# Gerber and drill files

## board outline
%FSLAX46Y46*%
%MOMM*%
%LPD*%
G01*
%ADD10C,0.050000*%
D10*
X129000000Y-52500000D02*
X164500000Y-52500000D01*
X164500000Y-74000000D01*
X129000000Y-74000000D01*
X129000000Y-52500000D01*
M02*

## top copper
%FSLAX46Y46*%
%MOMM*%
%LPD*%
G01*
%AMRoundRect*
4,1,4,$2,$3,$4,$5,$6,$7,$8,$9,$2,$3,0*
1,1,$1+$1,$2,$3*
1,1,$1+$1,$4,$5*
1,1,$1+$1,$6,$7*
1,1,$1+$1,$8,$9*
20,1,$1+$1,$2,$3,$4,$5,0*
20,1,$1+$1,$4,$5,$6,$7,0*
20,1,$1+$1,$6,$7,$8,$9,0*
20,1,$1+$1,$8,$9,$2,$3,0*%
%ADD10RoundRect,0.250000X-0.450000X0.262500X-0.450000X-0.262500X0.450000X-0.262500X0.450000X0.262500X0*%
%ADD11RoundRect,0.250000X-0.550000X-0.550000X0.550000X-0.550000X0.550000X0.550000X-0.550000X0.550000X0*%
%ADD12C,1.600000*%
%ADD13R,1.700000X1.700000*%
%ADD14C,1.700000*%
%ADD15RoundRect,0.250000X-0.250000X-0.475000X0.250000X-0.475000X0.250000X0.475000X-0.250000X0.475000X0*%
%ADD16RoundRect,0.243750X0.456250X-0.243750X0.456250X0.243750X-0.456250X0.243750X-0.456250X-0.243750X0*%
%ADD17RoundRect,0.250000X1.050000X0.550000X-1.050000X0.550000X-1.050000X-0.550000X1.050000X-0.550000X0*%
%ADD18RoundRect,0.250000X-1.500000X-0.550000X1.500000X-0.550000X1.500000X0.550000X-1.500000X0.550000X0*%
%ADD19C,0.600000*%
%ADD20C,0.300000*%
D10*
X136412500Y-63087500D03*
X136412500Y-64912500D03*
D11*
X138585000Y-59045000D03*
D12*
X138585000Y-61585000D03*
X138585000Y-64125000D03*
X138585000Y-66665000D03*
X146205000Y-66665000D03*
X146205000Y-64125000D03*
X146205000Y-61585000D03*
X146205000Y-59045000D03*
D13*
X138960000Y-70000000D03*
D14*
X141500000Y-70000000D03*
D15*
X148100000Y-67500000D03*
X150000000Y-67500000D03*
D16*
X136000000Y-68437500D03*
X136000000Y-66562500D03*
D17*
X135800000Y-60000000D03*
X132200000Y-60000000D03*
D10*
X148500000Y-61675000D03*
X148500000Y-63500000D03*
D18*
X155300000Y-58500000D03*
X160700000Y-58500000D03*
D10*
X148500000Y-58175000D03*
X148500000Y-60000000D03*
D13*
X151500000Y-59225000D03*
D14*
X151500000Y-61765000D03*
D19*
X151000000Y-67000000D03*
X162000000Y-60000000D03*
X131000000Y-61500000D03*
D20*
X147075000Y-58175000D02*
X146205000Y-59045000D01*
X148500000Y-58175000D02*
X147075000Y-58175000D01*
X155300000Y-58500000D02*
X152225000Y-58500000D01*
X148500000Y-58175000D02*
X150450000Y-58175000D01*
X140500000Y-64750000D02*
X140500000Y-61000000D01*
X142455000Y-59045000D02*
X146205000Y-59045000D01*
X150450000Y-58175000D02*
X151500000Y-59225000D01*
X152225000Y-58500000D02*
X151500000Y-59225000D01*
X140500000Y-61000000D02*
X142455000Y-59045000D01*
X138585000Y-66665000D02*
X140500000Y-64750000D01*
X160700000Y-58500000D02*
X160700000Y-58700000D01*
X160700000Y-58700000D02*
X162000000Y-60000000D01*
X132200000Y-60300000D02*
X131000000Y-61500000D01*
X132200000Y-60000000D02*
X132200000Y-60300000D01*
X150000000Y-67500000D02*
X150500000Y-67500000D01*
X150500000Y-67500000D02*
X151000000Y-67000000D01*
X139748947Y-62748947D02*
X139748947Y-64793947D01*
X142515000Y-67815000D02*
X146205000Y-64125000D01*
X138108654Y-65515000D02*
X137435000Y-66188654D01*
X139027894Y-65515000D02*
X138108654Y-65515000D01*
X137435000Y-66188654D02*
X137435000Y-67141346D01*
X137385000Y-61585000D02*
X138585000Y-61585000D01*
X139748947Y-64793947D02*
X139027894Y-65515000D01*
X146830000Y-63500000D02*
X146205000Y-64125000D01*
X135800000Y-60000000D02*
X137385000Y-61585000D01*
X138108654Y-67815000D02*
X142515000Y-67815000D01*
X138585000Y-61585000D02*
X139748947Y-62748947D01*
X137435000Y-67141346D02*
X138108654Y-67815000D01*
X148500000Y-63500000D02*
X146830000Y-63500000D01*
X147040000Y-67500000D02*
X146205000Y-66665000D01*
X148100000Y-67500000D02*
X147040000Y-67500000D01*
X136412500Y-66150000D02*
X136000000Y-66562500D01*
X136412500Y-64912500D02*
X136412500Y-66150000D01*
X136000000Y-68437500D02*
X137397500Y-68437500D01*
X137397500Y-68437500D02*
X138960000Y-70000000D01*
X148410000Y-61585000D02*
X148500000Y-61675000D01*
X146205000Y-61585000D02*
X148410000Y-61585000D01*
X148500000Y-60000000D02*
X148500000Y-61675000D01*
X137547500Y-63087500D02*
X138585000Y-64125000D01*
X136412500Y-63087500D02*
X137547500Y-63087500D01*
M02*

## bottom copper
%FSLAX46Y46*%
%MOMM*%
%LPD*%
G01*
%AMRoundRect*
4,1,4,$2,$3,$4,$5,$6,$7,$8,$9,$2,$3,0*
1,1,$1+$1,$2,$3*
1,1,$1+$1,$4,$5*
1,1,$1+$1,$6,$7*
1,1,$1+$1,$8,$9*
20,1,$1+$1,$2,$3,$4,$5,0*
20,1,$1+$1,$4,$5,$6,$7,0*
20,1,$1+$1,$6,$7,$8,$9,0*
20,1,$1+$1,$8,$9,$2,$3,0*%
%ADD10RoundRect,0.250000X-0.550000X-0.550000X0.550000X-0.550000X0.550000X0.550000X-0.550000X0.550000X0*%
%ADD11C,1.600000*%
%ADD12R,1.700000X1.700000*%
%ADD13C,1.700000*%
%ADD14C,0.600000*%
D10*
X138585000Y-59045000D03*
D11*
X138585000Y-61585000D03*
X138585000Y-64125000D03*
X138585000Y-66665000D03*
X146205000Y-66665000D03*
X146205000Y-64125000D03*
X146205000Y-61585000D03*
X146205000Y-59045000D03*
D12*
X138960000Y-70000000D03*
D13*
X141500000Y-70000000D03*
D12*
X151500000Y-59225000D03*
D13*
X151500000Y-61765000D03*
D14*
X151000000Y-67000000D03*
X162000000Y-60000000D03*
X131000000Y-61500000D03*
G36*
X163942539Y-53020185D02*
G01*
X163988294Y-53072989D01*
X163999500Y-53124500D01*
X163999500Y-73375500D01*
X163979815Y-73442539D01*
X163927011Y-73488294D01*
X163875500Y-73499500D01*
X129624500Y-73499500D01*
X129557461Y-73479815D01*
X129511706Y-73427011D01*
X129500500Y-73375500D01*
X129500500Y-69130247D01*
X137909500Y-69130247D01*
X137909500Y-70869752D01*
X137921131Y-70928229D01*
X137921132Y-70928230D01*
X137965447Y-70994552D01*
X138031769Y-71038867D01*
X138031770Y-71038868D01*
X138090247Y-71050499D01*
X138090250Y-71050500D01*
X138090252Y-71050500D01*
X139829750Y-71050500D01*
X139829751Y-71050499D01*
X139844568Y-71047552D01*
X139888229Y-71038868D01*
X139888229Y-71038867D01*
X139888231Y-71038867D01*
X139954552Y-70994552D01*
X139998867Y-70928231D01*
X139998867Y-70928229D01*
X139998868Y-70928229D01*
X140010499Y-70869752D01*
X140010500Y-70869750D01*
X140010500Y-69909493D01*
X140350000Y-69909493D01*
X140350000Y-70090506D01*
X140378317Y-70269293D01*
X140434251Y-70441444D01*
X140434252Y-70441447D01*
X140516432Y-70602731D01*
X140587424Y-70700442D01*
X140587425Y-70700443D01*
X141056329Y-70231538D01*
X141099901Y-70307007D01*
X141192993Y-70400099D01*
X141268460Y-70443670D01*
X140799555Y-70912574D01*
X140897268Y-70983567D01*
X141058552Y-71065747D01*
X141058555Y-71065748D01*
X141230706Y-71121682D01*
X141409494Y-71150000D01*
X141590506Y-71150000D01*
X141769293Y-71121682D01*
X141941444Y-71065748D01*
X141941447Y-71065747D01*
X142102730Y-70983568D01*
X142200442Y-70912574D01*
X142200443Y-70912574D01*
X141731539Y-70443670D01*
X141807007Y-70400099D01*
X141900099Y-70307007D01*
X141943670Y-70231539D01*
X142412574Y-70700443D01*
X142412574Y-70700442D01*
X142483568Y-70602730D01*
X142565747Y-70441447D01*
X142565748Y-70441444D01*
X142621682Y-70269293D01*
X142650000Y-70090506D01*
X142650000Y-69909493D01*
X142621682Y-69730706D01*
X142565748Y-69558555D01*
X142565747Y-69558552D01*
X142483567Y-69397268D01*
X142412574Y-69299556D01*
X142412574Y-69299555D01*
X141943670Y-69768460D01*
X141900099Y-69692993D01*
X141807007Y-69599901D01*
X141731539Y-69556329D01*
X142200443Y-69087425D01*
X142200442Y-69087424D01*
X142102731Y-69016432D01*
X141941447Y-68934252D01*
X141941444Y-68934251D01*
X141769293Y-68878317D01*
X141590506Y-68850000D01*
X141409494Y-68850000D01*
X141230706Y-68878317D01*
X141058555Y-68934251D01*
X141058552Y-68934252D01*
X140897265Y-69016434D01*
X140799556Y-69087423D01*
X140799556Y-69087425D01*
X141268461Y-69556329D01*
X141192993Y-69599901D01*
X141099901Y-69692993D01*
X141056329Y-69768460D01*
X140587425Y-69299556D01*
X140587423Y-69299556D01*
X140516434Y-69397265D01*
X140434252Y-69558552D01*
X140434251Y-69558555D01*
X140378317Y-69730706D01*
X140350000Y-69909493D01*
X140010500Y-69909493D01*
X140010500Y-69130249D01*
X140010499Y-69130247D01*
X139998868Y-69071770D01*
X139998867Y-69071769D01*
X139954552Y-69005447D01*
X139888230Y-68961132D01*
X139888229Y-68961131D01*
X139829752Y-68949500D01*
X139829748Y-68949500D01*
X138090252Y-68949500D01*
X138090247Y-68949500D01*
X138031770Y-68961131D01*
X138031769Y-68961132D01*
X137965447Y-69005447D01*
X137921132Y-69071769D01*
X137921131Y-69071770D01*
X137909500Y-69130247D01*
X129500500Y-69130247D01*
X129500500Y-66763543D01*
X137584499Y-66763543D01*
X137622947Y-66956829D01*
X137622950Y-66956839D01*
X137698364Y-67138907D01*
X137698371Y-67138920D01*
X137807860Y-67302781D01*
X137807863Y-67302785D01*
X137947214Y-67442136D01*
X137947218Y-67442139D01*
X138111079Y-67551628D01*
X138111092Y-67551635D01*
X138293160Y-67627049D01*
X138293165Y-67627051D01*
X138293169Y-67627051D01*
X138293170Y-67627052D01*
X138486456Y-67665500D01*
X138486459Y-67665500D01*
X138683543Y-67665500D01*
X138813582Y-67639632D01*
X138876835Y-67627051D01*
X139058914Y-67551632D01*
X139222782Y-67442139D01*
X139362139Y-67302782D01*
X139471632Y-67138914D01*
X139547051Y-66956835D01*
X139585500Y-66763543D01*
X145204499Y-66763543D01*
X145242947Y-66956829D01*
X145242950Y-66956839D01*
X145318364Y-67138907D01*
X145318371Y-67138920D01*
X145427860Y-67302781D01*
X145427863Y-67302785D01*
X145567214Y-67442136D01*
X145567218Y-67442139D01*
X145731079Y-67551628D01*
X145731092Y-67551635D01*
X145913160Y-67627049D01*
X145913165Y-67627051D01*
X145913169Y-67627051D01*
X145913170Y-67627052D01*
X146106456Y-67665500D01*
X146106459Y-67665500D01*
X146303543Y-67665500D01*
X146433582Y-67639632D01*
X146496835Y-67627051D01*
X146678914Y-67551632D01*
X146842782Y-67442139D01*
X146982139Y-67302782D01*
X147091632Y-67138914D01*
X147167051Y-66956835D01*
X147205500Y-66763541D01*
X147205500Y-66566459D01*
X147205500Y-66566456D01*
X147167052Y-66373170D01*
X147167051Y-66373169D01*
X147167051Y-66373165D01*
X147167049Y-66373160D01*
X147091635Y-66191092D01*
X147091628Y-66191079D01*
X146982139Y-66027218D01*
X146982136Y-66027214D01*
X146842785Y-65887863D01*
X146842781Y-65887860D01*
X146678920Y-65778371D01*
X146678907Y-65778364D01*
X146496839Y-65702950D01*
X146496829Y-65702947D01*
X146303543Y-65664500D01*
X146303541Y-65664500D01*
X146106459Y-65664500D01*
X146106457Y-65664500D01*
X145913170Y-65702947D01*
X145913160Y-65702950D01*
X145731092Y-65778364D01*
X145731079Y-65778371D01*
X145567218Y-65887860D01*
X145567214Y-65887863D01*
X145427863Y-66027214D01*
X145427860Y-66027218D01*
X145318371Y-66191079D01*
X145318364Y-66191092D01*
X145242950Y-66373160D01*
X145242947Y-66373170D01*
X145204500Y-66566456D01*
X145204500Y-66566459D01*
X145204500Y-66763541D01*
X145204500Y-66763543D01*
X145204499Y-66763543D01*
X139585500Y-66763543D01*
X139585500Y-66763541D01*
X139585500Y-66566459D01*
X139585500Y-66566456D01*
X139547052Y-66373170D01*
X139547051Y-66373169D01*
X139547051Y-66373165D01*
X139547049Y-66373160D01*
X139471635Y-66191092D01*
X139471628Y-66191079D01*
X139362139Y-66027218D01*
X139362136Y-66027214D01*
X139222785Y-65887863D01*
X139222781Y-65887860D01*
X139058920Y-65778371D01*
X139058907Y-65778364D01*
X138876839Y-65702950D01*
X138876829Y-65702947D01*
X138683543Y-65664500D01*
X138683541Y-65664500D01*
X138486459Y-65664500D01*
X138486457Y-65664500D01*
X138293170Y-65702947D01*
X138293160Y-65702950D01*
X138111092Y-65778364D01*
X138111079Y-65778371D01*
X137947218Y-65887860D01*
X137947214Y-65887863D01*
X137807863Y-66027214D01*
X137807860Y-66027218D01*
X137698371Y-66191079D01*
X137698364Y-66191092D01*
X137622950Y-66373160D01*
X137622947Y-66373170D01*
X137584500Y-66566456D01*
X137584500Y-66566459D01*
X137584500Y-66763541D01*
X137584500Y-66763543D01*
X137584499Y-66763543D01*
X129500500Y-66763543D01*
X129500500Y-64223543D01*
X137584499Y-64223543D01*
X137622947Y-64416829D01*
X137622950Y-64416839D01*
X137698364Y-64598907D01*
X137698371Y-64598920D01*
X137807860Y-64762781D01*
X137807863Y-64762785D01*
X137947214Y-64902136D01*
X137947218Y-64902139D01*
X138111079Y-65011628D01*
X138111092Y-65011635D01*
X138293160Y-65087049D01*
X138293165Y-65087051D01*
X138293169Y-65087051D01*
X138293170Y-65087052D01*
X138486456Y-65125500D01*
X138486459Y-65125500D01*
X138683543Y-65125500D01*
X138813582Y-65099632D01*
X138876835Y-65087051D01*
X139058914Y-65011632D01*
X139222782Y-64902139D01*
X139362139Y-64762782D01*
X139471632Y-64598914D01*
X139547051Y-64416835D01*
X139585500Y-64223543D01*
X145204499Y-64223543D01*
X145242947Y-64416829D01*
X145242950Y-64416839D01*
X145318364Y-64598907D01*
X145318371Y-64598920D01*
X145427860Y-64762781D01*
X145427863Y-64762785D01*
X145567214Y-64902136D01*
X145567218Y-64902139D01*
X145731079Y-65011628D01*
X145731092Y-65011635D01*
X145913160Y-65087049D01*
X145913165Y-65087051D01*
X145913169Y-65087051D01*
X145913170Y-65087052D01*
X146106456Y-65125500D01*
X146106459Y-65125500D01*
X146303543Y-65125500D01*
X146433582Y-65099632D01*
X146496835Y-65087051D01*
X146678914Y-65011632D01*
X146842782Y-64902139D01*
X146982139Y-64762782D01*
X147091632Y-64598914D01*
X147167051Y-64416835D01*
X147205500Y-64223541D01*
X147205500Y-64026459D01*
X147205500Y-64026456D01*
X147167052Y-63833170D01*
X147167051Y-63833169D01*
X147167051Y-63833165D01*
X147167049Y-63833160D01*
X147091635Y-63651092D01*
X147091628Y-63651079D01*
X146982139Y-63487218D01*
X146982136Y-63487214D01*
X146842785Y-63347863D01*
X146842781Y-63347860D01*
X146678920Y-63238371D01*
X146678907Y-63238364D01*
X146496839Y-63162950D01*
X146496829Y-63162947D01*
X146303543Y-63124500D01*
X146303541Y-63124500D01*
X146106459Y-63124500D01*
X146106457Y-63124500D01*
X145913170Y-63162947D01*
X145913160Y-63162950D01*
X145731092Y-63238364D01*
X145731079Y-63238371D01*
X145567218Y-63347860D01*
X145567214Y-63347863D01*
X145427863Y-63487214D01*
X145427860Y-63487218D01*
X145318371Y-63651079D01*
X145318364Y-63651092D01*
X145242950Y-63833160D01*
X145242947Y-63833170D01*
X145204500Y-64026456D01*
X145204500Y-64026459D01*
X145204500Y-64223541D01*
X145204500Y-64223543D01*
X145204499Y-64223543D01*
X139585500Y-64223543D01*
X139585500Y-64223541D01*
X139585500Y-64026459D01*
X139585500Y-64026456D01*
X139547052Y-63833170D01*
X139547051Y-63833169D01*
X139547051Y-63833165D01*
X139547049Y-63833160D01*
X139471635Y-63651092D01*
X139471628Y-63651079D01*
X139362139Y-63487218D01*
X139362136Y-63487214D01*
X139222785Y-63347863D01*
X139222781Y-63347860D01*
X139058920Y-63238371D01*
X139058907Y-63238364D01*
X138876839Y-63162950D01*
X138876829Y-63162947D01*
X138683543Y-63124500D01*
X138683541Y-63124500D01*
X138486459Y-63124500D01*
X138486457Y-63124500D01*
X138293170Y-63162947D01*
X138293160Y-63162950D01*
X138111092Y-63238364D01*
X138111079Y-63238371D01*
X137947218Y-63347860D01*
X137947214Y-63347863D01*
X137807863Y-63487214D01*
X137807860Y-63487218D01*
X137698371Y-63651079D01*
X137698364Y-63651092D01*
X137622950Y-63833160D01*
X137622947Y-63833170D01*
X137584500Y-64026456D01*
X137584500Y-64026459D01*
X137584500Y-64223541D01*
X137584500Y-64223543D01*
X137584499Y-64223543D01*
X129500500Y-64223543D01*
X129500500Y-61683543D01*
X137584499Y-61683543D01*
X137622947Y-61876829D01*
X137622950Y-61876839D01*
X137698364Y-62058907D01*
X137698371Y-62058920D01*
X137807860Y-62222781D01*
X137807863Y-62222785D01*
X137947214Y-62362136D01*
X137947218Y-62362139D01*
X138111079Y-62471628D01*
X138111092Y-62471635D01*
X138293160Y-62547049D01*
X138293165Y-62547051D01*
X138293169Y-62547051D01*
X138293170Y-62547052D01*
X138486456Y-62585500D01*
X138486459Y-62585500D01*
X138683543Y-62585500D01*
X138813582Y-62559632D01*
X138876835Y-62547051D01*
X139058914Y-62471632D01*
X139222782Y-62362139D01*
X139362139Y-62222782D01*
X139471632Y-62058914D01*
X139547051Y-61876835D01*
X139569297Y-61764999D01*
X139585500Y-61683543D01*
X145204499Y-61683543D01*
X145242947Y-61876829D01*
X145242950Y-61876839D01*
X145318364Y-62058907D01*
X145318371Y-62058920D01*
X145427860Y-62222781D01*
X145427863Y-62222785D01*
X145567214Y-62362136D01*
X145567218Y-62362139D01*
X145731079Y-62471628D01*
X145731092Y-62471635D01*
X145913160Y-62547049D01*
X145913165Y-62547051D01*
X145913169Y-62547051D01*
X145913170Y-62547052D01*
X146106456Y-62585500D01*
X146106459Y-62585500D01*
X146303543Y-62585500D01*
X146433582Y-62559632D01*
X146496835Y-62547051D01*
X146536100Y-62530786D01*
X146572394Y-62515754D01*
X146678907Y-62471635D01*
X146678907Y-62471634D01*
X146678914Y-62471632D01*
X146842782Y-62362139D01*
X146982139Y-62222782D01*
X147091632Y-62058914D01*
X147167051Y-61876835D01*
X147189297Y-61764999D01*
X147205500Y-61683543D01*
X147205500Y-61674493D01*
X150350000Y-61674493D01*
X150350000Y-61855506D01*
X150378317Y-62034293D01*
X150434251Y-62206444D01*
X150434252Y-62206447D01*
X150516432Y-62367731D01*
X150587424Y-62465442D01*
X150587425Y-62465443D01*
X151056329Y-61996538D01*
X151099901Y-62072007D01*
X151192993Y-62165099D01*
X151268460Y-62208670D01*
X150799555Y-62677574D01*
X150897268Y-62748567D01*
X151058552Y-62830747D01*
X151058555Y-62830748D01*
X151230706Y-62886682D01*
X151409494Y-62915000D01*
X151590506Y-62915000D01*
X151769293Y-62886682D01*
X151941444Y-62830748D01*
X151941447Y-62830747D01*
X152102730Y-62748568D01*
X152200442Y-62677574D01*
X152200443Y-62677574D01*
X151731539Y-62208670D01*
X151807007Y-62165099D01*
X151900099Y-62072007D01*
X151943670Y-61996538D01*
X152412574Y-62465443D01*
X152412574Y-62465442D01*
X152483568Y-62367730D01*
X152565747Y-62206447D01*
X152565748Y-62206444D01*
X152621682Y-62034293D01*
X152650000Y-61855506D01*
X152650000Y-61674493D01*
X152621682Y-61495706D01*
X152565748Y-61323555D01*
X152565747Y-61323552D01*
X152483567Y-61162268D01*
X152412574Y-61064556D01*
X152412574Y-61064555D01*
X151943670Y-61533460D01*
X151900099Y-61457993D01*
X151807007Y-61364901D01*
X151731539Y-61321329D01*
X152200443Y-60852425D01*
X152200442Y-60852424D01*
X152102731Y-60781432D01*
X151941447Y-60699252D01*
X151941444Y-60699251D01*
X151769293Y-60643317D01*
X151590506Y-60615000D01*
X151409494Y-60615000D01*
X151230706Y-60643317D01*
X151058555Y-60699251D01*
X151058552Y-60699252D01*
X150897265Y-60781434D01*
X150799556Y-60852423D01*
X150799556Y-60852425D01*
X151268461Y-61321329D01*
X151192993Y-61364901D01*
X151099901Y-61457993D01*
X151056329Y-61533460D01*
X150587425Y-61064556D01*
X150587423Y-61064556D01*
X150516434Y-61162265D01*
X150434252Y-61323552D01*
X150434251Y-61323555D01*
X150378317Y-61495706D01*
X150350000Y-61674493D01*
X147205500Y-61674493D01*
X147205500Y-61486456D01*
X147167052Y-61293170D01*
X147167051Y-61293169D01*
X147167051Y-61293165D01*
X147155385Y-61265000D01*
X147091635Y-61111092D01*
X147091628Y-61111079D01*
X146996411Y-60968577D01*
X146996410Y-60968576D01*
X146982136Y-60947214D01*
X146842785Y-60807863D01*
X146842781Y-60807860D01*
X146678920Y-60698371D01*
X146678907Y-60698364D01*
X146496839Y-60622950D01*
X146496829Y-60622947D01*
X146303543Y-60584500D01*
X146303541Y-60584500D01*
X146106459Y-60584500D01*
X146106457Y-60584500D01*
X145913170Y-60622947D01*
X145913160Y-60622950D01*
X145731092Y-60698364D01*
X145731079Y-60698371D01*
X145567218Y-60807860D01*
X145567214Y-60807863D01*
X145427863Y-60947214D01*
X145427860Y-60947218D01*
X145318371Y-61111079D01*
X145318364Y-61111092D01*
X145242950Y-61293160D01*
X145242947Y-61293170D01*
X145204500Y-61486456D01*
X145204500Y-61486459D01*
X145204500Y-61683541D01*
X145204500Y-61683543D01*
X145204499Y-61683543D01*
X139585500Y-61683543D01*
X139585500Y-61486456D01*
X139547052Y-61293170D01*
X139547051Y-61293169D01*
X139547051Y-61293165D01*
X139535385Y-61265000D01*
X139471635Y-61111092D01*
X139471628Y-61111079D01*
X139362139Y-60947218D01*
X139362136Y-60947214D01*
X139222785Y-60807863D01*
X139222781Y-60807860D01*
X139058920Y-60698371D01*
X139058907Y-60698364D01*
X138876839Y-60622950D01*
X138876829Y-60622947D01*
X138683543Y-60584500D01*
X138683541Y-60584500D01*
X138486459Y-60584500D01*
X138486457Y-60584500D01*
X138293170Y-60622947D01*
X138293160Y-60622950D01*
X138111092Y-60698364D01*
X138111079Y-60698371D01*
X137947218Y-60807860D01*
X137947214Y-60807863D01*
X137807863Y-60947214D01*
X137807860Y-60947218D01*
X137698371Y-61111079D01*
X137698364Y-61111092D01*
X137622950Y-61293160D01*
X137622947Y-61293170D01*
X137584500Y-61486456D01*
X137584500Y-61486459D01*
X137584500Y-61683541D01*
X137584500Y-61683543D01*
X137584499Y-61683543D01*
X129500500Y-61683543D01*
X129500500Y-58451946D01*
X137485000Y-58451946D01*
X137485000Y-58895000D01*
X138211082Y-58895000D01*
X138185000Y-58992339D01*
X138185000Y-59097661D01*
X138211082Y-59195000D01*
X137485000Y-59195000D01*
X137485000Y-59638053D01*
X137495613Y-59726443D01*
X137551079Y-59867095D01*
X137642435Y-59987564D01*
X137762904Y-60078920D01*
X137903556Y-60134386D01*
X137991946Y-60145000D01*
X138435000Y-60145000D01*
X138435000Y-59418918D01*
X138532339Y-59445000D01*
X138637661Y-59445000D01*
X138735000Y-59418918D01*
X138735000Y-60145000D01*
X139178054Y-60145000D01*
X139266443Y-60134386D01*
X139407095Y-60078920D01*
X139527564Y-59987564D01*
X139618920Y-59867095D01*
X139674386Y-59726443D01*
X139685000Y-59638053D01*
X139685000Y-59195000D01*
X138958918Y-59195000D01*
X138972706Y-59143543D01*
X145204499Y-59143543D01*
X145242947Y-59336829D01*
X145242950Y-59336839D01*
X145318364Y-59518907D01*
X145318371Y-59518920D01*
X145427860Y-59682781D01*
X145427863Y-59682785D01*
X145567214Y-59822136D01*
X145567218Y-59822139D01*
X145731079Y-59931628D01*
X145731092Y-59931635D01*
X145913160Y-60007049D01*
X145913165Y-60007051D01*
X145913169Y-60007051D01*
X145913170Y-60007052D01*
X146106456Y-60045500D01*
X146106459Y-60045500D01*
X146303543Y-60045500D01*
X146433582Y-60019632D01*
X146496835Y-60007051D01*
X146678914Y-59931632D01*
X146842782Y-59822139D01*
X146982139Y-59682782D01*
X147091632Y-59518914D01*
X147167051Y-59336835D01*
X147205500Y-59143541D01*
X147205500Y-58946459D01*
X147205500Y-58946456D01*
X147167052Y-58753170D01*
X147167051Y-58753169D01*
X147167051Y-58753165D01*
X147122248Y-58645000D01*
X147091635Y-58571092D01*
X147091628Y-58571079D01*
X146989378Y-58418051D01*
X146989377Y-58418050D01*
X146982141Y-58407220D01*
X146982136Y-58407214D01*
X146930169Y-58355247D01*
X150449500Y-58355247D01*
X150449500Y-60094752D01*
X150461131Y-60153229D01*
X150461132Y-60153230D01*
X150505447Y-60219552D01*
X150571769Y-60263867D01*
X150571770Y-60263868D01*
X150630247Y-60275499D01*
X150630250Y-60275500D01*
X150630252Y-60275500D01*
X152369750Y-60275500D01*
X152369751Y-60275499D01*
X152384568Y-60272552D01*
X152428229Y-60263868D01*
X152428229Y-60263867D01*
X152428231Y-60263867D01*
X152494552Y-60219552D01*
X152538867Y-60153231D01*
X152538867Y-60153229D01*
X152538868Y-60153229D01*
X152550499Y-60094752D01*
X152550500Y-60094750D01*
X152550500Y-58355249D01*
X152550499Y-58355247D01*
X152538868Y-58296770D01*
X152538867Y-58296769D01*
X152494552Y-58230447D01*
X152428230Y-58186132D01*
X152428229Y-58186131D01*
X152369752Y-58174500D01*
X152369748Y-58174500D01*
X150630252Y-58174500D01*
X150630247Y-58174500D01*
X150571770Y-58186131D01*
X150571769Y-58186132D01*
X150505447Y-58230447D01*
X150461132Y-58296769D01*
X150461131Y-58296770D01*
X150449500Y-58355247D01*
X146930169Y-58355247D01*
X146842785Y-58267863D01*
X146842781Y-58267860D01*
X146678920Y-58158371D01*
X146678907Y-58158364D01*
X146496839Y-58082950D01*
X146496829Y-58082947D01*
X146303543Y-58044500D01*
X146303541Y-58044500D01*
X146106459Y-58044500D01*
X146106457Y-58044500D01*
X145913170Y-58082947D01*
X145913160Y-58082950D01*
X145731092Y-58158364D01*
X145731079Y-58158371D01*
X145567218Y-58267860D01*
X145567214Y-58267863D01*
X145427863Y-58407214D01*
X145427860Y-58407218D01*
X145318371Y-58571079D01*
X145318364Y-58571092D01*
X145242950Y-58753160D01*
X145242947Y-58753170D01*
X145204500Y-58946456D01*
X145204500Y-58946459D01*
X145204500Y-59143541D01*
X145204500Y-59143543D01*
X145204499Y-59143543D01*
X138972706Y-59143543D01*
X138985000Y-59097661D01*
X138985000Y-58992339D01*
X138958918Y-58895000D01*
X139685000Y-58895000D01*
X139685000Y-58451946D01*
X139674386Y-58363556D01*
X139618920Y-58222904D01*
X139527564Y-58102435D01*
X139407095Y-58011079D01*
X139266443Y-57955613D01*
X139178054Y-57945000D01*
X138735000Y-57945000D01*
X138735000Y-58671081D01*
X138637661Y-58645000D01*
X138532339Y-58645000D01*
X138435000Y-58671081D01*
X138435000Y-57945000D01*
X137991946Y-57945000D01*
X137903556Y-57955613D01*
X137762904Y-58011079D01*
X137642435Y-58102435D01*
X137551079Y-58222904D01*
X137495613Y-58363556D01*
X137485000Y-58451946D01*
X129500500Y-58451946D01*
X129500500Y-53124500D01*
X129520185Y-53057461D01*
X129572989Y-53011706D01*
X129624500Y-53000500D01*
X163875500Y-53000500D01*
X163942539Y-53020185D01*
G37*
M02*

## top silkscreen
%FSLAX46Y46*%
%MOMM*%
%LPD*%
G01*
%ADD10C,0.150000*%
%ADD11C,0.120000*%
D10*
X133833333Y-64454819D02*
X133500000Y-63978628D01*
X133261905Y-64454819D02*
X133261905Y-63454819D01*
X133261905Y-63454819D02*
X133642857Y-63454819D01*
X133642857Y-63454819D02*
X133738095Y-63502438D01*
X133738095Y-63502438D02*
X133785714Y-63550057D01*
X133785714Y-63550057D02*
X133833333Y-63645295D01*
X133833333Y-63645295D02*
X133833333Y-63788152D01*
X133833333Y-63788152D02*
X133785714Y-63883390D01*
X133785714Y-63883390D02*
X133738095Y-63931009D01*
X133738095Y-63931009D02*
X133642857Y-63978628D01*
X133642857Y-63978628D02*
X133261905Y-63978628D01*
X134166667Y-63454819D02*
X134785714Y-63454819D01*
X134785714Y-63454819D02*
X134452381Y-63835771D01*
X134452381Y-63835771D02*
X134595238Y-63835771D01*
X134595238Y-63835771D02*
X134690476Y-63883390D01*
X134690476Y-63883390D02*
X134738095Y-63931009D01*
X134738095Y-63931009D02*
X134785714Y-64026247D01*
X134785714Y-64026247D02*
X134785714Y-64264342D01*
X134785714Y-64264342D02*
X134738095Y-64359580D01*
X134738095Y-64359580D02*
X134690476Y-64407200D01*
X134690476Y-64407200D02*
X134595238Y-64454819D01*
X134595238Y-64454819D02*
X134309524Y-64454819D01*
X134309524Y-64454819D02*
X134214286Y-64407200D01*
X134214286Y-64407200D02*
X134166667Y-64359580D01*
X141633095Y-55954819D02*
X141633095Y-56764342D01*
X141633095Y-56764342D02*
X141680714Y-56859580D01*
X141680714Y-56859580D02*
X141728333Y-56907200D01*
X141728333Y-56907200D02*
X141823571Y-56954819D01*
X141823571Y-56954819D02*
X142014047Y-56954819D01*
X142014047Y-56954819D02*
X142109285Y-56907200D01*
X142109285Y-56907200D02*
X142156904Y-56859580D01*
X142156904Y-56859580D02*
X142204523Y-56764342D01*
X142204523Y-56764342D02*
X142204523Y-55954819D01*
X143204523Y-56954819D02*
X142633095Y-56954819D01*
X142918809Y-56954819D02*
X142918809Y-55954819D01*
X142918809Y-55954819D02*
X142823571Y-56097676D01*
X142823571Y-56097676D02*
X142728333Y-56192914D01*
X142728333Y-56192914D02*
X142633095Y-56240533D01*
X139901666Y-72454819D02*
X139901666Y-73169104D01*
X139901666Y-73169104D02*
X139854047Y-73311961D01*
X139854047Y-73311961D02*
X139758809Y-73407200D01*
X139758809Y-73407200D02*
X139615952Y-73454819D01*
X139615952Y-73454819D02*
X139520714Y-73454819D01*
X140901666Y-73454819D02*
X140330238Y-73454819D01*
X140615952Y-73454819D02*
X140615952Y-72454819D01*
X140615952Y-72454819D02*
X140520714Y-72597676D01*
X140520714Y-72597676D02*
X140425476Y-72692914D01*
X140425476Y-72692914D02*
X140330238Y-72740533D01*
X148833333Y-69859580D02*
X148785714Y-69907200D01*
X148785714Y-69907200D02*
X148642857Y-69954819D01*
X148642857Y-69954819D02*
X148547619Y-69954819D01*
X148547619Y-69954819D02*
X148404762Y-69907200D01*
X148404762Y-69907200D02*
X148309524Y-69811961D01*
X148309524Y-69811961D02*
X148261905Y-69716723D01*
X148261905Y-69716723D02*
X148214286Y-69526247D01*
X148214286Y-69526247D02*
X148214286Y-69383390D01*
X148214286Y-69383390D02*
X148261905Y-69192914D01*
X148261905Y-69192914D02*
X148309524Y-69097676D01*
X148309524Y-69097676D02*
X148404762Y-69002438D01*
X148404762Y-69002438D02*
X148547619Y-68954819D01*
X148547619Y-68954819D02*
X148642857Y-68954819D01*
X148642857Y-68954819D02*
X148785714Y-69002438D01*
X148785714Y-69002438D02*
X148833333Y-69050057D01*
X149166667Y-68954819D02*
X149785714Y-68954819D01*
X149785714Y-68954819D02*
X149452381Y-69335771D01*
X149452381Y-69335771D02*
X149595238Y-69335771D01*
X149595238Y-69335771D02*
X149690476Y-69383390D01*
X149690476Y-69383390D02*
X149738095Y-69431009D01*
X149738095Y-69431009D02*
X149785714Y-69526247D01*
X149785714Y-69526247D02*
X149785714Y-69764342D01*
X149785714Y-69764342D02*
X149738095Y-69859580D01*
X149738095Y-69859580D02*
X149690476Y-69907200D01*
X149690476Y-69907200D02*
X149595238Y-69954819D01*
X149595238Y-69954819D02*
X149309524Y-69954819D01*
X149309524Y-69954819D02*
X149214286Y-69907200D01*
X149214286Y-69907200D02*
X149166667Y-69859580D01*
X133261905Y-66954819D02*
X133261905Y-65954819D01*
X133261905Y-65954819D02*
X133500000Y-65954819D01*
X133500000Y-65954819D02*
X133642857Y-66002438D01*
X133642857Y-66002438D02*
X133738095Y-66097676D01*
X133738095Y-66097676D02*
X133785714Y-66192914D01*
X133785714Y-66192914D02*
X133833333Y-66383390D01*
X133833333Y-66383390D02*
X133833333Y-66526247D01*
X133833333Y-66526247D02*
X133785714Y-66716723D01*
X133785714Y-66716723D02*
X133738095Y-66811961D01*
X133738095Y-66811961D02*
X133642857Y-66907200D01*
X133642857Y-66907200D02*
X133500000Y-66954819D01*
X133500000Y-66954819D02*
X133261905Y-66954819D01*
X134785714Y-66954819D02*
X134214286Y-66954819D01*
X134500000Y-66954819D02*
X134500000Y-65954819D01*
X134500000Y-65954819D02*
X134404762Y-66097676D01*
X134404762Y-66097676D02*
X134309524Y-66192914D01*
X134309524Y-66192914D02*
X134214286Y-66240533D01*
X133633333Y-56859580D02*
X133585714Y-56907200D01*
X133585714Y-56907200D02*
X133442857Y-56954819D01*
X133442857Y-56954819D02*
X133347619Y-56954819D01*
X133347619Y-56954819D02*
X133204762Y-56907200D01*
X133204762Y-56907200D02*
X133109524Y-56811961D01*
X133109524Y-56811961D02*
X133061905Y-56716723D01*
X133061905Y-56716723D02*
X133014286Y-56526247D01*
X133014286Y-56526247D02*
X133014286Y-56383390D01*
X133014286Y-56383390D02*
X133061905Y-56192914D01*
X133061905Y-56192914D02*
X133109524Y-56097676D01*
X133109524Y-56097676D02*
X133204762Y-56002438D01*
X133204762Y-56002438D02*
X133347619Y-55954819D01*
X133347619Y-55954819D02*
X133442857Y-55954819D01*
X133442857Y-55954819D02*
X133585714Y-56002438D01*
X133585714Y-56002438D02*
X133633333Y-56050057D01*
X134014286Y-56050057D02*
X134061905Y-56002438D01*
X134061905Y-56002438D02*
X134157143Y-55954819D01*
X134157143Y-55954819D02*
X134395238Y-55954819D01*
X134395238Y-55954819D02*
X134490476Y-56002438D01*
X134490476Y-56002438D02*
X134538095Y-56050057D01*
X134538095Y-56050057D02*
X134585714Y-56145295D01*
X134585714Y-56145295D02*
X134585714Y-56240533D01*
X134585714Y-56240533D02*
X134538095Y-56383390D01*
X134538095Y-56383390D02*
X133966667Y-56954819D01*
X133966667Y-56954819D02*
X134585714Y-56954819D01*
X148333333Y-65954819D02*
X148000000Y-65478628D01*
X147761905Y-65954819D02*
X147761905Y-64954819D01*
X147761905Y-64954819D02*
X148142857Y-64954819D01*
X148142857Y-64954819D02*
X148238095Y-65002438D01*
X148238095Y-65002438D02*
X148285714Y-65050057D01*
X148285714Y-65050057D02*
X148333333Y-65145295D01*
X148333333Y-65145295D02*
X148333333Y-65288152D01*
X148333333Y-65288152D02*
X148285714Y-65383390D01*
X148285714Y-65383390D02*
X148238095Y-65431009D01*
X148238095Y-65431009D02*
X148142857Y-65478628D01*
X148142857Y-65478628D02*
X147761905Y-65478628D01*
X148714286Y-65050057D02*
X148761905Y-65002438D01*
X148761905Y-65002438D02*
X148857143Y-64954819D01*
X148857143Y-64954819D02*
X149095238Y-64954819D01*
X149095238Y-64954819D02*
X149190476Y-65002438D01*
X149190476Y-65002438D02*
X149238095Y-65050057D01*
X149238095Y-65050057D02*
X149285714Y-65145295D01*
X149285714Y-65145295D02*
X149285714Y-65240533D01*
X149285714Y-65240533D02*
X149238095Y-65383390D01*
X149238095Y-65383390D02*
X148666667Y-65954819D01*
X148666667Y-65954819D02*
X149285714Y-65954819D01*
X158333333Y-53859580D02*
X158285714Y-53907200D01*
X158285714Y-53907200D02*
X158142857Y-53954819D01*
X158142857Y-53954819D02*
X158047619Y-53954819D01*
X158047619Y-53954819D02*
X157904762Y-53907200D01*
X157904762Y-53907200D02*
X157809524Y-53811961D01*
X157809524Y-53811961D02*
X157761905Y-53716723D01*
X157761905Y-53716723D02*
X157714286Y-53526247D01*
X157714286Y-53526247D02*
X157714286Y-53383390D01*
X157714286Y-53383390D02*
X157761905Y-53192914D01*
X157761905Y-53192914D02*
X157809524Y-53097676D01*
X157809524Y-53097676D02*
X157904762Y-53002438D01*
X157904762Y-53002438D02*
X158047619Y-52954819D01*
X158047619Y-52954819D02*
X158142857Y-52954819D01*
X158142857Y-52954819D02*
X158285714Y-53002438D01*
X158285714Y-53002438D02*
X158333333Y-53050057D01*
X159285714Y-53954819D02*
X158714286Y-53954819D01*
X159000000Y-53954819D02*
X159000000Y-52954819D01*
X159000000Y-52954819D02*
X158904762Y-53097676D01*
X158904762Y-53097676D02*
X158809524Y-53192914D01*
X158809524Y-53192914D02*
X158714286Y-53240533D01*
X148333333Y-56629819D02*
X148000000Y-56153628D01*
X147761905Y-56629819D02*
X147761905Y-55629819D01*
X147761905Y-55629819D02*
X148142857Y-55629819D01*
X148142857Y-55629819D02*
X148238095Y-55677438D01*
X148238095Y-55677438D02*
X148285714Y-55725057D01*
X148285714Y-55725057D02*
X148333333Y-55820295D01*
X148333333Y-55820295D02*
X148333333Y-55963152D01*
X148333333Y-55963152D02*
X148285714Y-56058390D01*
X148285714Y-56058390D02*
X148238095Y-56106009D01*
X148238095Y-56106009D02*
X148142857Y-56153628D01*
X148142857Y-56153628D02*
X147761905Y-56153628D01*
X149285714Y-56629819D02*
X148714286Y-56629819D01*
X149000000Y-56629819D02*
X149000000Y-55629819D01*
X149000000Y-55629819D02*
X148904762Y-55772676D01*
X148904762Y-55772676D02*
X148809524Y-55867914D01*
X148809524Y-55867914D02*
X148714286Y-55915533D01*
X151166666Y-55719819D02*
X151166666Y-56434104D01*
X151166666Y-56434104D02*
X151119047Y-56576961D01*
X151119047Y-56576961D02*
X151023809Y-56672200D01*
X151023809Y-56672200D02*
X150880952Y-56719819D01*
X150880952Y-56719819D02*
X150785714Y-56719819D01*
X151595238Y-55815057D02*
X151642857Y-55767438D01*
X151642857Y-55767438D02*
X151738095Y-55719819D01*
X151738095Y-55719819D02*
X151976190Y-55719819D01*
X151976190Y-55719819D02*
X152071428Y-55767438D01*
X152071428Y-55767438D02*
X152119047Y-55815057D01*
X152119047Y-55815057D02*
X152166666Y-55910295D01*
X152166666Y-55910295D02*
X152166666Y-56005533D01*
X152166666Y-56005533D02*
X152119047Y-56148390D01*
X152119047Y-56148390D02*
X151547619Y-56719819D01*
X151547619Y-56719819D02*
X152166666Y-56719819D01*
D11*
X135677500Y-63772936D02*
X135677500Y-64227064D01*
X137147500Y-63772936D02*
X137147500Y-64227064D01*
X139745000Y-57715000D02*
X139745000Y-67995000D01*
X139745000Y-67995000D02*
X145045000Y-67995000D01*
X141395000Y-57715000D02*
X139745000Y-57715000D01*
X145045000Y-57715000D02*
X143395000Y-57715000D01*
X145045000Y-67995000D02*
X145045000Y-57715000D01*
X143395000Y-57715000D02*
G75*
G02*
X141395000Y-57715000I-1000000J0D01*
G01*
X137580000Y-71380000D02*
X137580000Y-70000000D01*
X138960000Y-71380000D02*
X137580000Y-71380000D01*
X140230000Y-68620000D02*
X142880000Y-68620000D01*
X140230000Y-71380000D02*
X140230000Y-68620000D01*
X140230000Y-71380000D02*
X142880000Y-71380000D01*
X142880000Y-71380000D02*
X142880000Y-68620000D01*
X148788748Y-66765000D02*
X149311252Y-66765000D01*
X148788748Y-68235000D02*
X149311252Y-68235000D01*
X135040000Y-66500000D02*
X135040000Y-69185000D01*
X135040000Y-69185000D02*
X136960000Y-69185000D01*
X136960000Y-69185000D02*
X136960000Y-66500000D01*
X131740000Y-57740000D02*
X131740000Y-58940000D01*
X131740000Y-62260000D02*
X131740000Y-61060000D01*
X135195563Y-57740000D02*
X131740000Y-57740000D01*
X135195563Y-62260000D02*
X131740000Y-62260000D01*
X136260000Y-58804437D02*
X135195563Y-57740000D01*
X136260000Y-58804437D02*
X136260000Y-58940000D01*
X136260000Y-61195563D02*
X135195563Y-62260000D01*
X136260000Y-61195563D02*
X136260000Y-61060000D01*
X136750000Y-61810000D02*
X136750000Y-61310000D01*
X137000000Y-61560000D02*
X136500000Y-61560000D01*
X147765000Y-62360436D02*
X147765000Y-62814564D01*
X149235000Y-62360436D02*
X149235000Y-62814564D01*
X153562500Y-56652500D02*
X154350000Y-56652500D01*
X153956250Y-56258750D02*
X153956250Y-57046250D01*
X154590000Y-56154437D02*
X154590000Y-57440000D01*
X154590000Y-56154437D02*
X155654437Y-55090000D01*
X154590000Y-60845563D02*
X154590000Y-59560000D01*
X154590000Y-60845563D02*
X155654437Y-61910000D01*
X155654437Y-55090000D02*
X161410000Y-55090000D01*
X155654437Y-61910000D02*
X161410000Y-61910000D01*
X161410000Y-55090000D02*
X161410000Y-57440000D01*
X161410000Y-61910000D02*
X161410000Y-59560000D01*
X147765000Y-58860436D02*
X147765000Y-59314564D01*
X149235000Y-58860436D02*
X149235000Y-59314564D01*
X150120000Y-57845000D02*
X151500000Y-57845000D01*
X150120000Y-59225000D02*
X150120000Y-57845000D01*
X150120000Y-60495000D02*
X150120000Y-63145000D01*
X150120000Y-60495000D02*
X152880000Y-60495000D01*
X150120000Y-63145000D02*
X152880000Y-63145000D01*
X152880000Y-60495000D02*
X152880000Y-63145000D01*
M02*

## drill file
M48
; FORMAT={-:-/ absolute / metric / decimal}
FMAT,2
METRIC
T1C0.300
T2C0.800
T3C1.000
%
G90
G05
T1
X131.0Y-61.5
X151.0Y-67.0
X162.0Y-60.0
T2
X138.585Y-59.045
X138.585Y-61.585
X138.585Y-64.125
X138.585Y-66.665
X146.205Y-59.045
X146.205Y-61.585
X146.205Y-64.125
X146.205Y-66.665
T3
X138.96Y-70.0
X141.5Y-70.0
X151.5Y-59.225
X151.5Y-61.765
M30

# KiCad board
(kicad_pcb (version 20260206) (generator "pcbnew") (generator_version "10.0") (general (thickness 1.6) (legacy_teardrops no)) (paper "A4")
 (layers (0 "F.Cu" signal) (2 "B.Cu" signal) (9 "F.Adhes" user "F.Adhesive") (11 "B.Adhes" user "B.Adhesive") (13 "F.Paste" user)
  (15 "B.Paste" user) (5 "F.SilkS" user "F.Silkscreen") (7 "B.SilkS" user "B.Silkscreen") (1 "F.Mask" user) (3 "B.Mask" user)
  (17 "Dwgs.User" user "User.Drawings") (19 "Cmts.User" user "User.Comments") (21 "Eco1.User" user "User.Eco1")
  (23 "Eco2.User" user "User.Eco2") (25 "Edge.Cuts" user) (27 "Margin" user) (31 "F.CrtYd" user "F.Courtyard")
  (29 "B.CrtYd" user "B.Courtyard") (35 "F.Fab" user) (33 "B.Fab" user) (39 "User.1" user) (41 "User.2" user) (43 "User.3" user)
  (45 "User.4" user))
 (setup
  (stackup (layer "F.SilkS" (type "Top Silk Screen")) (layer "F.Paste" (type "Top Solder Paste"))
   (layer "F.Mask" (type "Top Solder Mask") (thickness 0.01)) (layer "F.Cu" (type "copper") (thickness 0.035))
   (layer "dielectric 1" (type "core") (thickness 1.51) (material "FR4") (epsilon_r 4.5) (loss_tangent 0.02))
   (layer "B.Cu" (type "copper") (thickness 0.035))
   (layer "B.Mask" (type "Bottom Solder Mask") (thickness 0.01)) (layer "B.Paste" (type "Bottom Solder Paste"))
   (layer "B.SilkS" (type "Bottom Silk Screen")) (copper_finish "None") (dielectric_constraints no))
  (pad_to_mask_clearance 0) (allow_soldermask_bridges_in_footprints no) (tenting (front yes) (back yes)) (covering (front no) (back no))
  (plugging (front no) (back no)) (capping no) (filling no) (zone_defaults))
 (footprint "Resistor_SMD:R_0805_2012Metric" (layer "F.Cu") (at 136.4125 64 -90)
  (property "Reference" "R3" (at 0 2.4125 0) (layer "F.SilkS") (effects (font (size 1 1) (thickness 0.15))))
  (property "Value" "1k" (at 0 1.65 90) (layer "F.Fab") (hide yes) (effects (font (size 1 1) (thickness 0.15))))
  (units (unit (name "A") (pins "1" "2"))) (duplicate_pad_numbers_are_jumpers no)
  (fp_line (start -0.227064 0.735) (end 0.227064 0.735) (stroke (width 0.12) (type solid)) (layer "F.SilkS"))
  (fp_line (start -0.227064 -0.735) (end 0.227064 -0.735) (stroke (width 0.12) (type solid)) (layer "F.SilkS"))
  (pad "1" smd roundrect (at -0.9125 0 270) (size 1.025 1.4) (layers "F.Cu" "F.Mask" "F.Paste") (roundrect_rratio 0.243902)
   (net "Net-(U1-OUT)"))
  (pad "2" smd roundrect (at 0.9125 0 270) (size 1.025 1.4) (layers "F.Cu" "F.Mask" "F.Paste") (roundrect_rratio 0.243902)
   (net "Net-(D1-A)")))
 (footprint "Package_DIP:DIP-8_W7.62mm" (layer "F.Cu") (at 138.585 59.045)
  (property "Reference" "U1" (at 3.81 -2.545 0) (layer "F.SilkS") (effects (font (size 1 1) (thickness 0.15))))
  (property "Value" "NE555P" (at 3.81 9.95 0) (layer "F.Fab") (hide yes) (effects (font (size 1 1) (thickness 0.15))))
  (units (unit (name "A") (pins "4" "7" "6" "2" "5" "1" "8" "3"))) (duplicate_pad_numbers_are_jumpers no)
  (fp_line (start 1.16 -1.33) (end 1.16 8.95) (stroke (width 0.12) (type solid)) (layer "F.SilkS"))
  (fp_line (start 1.16 8.95) (end 6.46 8.95) (stroke (width 0.12) (type solid)) (layer "F.SilkS"))
  (fp_line (start 2.81 -1.33) (end 1.16 -1.33) (stroke (width 0.12) (type solid)) (layer "F.SilkS"))
  (fp_line (start 6.46 -1.33) (end 4.81 -1.33) (stroke (width 0.12) (type solid)) (layer "F.SilkS"))
  (fp_line (start 6.46 8.95) (end 6.46 -1.33) (stroke (width 0.12) (type solid)) (layer "F.SilkS"))
  (fp_arc (start 4.81 -1.33) (mid 3.81 -0.33) (end 2.81 -1.33) (stroke (width 0.12) (type solid)) (layer "F.SilkS"))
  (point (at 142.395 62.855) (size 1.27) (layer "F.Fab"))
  (pad "1" thru_hole roundrect (at 0 0) (size 1.6 1.6) (drill 0.8) (layers "*.Cu" "*.Mask") (remove_unused_layers no)
   (roundrect_rratio 0.15625) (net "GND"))
  (pad "2" thru_hole circle (at 0 2.54) (size 1.6 1.6) (drill 0.8) (layers "*.Cu" "*.Mask") (remove_unused_layers no) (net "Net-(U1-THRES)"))
  (pad "3" thru_hole circle (at 0 5.08) (size 1.6 1.6) (drill 0.8) (layers "*.Cu" "*.Mask") (remove_unused_layers no) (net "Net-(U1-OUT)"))
  (pad "4" thru_hole circle (at 0 7.62) (size 1.6 1.6) (drill 0.8) (layers "*.Cu" "*.Mask") (remove_unused_layers no) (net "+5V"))
  (pad "5" thru_hole circle (at 7.62 7.62) (size 1.6 1.6) (drill 0.8) (layers "*.Cu" "*.Mask") (remove_unused_layers no)
   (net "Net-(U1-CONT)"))
  (pad "6" thru_hole circle (at 7.62 5.08) (size 1.6 1.6) (drill 0.8) (layers "*.Cu" "*.Mask") (remove_unused_layers no)
   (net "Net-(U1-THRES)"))
  (pad "7" thru_hole circle (at 7.62 2.54) (size 1.6 1.6) (drill 0.8) (layers "*.Cu" "*.Mask") (remove_unused_layers no)
   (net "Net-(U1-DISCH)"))
  (pad "8" thru_hole circle (at 7.62 0) (size 1.6 1.6) (drill 0.8) (layers "*.Cu" "*.Mask") (remove_unused_layers no) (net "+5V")))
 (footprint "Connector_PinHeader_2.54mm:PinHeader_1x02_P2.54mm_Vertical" (layer "F.Cu") (at 138.96 70 90)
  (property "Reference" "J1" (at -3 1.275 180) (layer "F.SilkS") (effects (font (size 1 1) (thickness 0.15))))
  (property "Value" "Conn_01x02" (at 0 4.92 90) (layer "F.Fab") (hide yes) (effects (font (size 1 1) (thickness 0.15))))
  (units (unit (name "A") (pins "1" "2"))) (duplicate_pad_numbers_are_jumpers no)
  (fp_line (start -1.38 -1.38) (end 0 -1.38) (stroke (width 0.12) (type solid)) (layer "F.SilkS"))
  (fp_line (start -1.38 0) (end -1.38 -1.38) (stroke (width 0.12) (type solid)) (layer "F.SilkS"))
  (fp_line (start 1.38 1.27) (end 1.38 3.92) (stroke (width 0.12) (type solid)) (layer "F.SilkS"))
  (fp_line (start -1.38 1.27) (end 1.38 1.27) (stroke (width 0.12) (type solid)) (layer "F.SilkS"))
  (fp_line (start -1.38 1.27) (end -1.38 3.92) (stroke (width 0.12) (type solid)) (layer "F.SilkS"))
  (fp_line (start -1.38 3.92) (end 1.38 3.92) (stroke (width 0.12) (type solid)) (layer "F.SilkS"))
  (pad "1" thru_hole rect (at 0 0 90) (size 1.7 1.7) (drill 1) (layers "*.Cu" "*.Mask") (remove_unused_layers no) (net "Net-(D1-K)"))
  (pad "2" thru_hole circle (at 0 2.54 90) (size 1.7 1.7) (drill 1) (layers "*.Cu" "*.Mask") (remove_unused_layers no) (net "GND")))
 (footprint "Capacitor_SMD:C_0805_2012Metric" (layer "F.Cu") (at 149.05 67.5)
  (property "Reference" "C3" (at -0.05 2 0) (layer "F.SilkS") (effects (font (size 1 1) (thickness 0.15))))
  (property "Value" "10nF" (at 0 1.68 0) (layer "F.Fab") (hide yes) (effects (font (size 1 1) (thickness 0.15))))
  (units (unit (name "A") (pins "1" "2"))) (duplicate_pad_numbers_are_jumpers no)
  (fp_line (start -0.261252 -0.735) (end 0.261252 -0.735) (stroke (width 0.12) (type solid)) (layer "F.SilkS"))
  (fp_line (start -0.261252 0.735) (end 0.261252 0.735) (stroke (width 0.12) (type solid)) (layer "F.SilkS"))
  (pad "1" smd roundrect (at -0.95 0) (size 1 1.45) (layers "F.Cu" "F.Mask" "F.Paste") (roundrect_rratio 0.25) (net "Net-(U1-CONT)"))
  (pad "2" smd roundrect (at 0.95 0) (size 1 1.45) (layers "F.Cu" "F.Mask" "F.Paste") (roundrect_rratio 0.25) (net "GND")))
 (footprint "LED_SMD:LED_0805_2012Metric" (layer "F.Cu") (at 136 67.5 90)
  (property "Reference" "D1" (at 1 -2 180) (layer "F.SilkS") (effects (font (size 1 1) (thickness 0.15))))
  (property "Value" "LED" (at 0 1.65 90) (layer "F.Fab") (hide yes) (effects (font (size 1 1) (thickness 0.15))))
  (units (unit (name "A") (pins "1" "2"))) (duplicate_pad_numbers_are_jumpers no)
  (fp_line (start 1 -0.96) (end -1.685 -0.96) (stroke (width 0.12) (type solid)) (layer "F.SilkS"))
  (fp_line (start -1.685 -0.96) (end -1.685 0.96) (stroke (width 0.12) (type solid)) (layer "F.SilkS"))
  (fp_line (start -1.685 0.96) (end 1 0.96) (stroke (width 0.12) (type solid)) (layer "F.SilkS"))
  (pad "1" smd roundrect (at -0.9375 0 90) (size 0.975 1.4) (layers "F.Cu" "F.Mask" "F.Paste") (roundrect_rratio 0.25) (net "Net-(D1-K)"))
  (pad "2" smd roundrect (at 0.9375 0 90) (size 0.975 1.4) (layers "F.Cu" "F.Mask" "F.Paste") (roundrect_rratio 0.25) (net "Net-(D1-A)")))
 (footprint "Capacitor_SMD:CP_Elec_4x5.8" (layer "F.Cu") (at 134 60 180)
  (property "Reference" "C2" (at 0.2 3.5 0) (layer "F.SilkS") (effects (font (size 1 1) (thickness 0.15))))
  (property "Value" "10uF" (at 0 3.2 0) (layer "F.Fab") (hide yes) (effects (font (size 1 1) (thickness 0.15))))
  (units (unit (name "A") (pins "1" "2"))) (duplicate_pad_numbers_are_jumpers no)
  (fp_line (start 2.26 2.26) (end 2.26 1.06) (stroke (width 0.12) (type solid)) (layer "F.SilkS"))
  (fp_line (start 2.26 -2.26) (end 2.26 -1.06) (stroke (width 0.12) (type solid)) (layer "F.SilkS"))
  (fp_line (start -1.195563 2.26) (end 2.26 2.26) (stroke (width 0.12) (type solid)) (layer "F.SilkS"))
  (fp_line (start -1.195563 -2.26) (end 2.26 -2.26) (stroke (width 0.12) (type solid)) (layer "F.SilkS"))
  (fp_line (start -2.26 1.195563) (end -1.195563 2.26) (stroke (width 0.12) (type solid)) (layer "F.SilkS"))
  (fp_line (start -2.26 1.195563) (end -2.26 1.06) (stroke (width 0.12) (type solid)) (layer "F.SilkS"))
  (fp_line (start -2.26 -1.195563) (end -1.195563 -2.26) (stroke (width 0.12) (type solid)) (layer "F.SilkS"))
  (fp_line (start -2.26 -1.195563) (end -2.26 -1.06) (stroke (width 0.12) (type solid)) (layer "F.SilkS"))
  (fp_line (start -2.75 -1.81) (end -2.75 -1.31) (stroke (width 0.12) (type solid)) (layer "F.SilkS"))
  (fp_line (start -3 -1.56) (end -2.5 -1.56) (stroke (width 0.12) (type solid)) (layer "F.SilkS"))
  (pad "1" smd roundrect (at -1.8 0 180) (size 2.6 1.6) (layers "F.Cu" "F.Mask" "F.Paste") (roundrect_rratio 0.15625) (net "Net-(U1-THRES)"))
  (pad "2" smd roundrect (at 1.8 0 180) (size 2.6 1.6) (layers "F.Cu" "F.Mask" "F.Paste") (roundrect_rratio 0.15625) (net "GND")))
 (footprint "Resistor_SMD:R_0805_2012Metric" (layer "F.Cu") (at 148.5 62.5875 -90)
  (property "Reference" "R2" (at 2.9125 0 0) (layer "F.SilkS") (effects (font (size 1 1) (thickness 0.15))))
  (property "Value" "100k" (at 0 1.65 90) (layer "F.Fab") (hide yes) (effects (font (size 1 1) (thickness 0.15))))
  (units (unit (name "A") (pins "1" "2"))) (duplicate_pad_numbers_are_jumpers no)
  (fp_line (start -0.227064 0.735) (end 0.227064 0.735) (stroke (width 0.12) (type solid)) (layer "F.SilkS"))
  (fp_line (start -0.227064 -0.735) (end 0.227064 -0.735) (stroke (width 0.12) (type solid)) (layer "F.SilkS"))
  (pad "1" smd roundrect (at -0.9125 0 270) (size 1.025 1.4) (layers "F.Cu" "F.Mask" "F.Paste") (roundrect_rratio 0.243902)
   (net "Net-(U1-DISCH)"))
  (pad "2" smd roundrect (at 0.9125 0 270) (size 1.025 1.4) (layers "F.Cu" "F.Mask" "F.Paste") (roundrect_rratio 0.243902)
   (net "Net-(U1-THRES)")))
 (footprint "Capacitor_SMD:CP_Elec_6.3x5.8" (layer "F.Cu") (at 158 58.5)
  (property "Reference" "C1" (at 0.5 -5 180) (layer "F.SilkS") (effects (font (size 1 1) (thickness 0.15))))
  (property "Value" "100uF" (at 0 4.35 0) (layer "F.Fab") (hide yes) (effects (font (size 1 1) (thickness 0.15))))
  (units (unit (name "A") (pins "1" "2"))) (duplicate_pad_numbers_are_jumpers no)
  (fp_line (start -4.4375 -1.8475) (end -3.65 -1.8475) (stroke (width 0.12) (type solid)) (layer "F.SilkS"))
  (fp_line (start -4.04375 -2.24125) (end -4.04375 -1.45375) (stroke (width 0.12) (type solid)) (layer "F.SilkS"))
  (fp_line (start -3.41 -2.345563) (end -3.41 -1.06) (stroke (width 0.12) (type solid)) (layer "F.SilkS"))
  (fp_line (start -3.41 -2.345563) (end -2.345563 -3.41) (stroke (width 0.12) (type solid)) (layer "F.SilkS"))
  (fp_line (start -3.41 2.345563) (end -3.41 1.06) (stroke (width 0.12) (type solid)) (layer "F.SilkS"))
  (fp_line (start -3.41 2.345563) (end -2.345563 3.41) (stroke (width 0.12) (type solid)) (layer "F.SilkS"))
  (fp_line (start -2.345563 -3.41) (end 3.41 -3.41) (stroke (width 0.12) (type solid)) (layer "F.SilkS"))
  (fp_line (start -2.345563 3.41) (end 3.41 3.41) (stroke (width 0.12) (type solid)) (layer "F.SilkS"))
  (fp_line (start 3.41 -3.41) (end 3.41 -1.06) (stroke (width 0.12) (type solid)) (layer "F.SilkS"))
  (fp_line (start 3.41 3.41) (end 3.41 1.06) (stroke (width 0.12) (type solid)) (layer "F.SilkS"))
  (pad "1" smd roundrect (at -2.7 0) (size 3.5 1.6) (layers "F.Cu" "F.Mask" "F.Paste") (roundrect_rratio 0.15625) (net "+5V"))
  (pad "2" smd roundrect (at 2.7 0) (size 3.5 1.6) (layers "F.Cu" "F.Mask" "F.Paste") (roundrect_rratio 0.15625) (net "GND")))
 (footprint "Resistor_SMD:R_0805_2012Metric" (layer "F.Cu") (at 148.5 59.0875 -90)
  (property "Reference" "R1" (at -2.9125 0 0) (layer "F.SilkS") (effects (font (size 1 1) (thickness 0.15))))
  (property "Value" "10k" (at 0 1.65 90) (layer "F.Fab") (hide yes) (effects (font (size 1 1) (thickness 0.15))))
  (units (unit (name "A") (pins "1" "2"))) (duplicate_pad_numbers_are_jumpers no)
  (fp_line (start -0.227064 0.735) (end 0.227064 0.735) (stroke (width 0.12) (type solid)) (layer "F.SilkS"))
  (fp_line (start -0.227064 -0.735) (end 0.227064 -0.735) (stroke (width 0.12) (type solid)) (layer "F.SilkS"))
  (pad "1" smd roundrect (at -0.9125 0 270) (size 1.025 1.4) (layers "F.Cu" "F.Mask" "F.Paste") (roundrect_rratio 0.243902) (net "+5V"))
  (pad "2" smd roundrect (at 0.9125 0 270) (size 1.025 1.4) (layers "F.Cu" "F.Mask" "F.Paste") (roundrect_rratio 0.243902)
   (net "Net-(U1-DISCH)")))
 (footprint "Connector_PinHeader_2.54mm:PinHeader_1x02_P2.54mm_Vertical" (layer "F.Cu") (at 151.5 59.225)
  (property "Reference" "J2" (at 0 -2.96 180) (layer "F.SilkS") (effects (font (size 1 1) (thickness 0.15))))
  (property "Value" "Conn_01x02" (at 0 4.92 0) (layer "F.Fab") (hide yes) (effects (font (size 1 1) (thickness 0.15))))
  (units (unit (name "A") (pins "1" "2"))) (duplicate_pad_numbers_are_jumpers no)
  (fp_line (start -1.38 -1.38) (end 0 -1.38) (stroke (width 0.12) (type solid)) (layer "F.SilkS"))
  (fp_line (start -1.38 0) (end -1.38 -1.38) (stroke (width 0.12) (type solid)) (layer "F.SilkS"))
  (fp_line (start -1.38 1.27) (end -1.38 3.92) (stroke (width 0.12) (type solid)) (layer "F.SilkS"))
  (fp_line (start -1.38 1.27) (end 1.38 1.27) (stroke (width 0.12) (type solid)) (layer "F.SilkS"))
  (fp_line (start -1.38 3.92) (end 1.38 3.92) (stroke (width 0.12) (type solid)) (layer "F.SilkS"))
  (fp_line (start 1.38 1.27) (end 1.38 3.92) (stroke (width 0.12) (type solid)) (layer "F.SilkS"))
  (pad "1" thru_hole rect (at 0 0) (size 1.7 1.7) (drill 1) (layers "*.Cu" "*.Mask") (remove_unused_layers no) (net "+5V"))
  (pad "2" thru_hole circle (at 0 2.54) (size 1.7 1.7) (drill 1) (layers "*.Cu" "*.Mask") (remove_unused_layers no) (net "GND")))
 (gr_rect (start 129 52.5) (end 164.5 74) (stroke (width 0.05) (type default)) (fill no) (layer "Edge.Cuts"))
 (segment (start 147.075 58.175) (end 146.205 59.045) (width 0.3) (layer "F.Cu") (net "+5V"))
 (segment (start 148.5 58.175) (end 147.075 58.175) (width 0.3) (layer "F.Cu") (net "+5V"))
 (segment (start 155.3 58.5) (end 152.225 58.5) (width 0.3) (layer "F.Cu") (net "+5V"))
 (segment (start 148.5 58.175) (end 150.45 58.175) (width 0.3) (layer "F.Cu") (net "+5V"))
 (segment (start 140.5 64.75) (end 140.5 61) (width 0.3) (layer "F.Cu") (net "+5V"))
 (segment (start 142.455 59.045) (end 146.205 59.045) (width 0.3) (layer "F.Cu") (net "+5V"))
 (segment (start 150.45 58.175) (end 151.5 59.225) (width 0.3) (layer "F.Cu") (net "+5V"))
 (segment (start 152.225 58.5) (end 151.5 59.225) (width 0.3) (layer "F.Cu") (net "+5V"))
 (segment (start 140.5 61) (end 142.455 59.045) (width 0.3) (layer "F.Cu") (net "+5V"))
 (segment (start 138.585 66.665) (end 140.5 64.75) (width 0.3) (layer "F.Cu") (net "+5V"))
 (segment (start 160.7 58.5) (end 160.7 58.7) (width 0.3) (layer "F.Cu") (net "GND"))
 (segment (start 160.7 58.7) (end 162 60) (width 0.3) (layer "F.Cu") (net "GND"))
 (segment (start 132.2 60.3) (end 131 61.5) (width 0.3) (layer "F.Cu") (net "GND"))
 (segment (start 132.2 60) (end 132.2 60.3) (width 0.3) (layer "F.Cu") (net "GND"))
 (segment (start 150 67.5) (end 150.5 67.5) (width 0.3) (layer "F.Cu") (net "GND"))
 (segment (start 150.5 67.5) (end 151 67) (width 0.3) (layer "F.Cu") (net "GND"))
 (via (at 151 67) (size 0.6) (drill 0.3) (layers "F.Cu" "B.Cu") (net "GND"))
 (via (at 162 60) (size 0.6) (drill 0.3) (layers "F.Cu" "B.Cu") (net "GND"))
 (via (at 131 61.5) (size 0.6) (drill 0.3) (layers "F.Cu" "B.Cu") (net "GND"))
 (segment (start 139.748947 62.748947) (end 139.748947 64.793947) (width 0.3) (layer "F.Cu") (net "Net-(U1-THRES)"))
 (segment (start 142.515 67.815) (end 146.205 64.125) (width 0.3) (layer "F.Cu") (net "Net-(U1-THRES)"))
 (segment (start 138.108654 65.515) (end 137.435 66.188654) (width 0.3) (layer "F.Cu") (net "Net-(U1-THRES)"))
 (segment (start 139.027894 65.515) (end 138.108654 65.515) (width 0.3) (layer "F.Cu") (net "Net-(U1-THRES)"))
 (segment (start 137.435 66.188654) (end 137.435 67.141346) (width 0.3) (layer "F.Cu") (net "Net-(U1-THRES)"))
 (segment (start 137.385 61.585) (end 138.585 61.585) (width 0.3) (layer "F.Cu") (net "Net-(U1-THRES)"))
 (segment (start 139.748947 64.793947) (end 139.027894 65.515) (width 0.3) (layer "F.Cu") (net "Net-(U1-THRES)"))
 (segment (start 146.83 63.5) (end 146.205 64.125) (width 0.3) (layer "F.Cu") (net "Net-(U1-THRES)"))
 (segment (start 135.8 60) (end 137.385 61.585) (width 0.3) (layer "F.Cu") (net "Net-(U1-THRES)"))
 (segment (start 138.108654 67.815) (end 142.515 67.815) (width 0.3) (layer "F.Cu") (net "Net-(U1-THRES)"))
 (segment (start 138.585 61.585) (end 139.748947 62.748947) (width 0.3) (layer "F.Cu") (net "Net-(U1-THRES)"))
 (segment (start 137.435 67.141346) (end 138.108654 67.815) (width 0.3) (layer "F.Cu") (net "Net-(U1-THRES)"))
 (segment (start 148.5 63.5) (end 146.83 63.5) (width 0.3) (layer "F.Cu") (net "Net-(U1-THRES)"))
 (segment (start 147.04 67.5) (end 146.205 66.665) (width 0.3) (layer "F.Cu") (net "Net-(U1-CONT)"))
 (segment (start 148.1 67.5) (end 147.04 67.5) (width 0.3) (layer "F.Cu") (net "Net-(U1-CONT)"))
 (segment (start 136.4125 66.15) (end 136 66.5625) (width 0.3) (layer "F.Cu") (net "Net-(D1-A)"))
 (segment (start 136.4125 64.9125) (end 136.4125 66.15) (width 0.3) (layer "F.Cu") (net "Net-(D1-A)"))
 (segment (start 136 68.4375) (end 137.3975 68.4375) (width 0.3) (layer "F.Cu") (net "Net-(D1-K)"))
 (segment (start 137.3975 68.4375) (end 138.96 70) (width 0.3) (layer "F.Cu") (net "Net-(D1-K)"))
 (segment (start 148.41 61.585) (end 148.5 61.675) (width 0.3) (layer "F.Cu") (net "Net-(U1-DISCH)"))
 (segment (start 146.205 61.585) (end 148.41 61.585) (width 0.3) (layer "F.Cu") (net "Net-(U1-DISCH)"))
 (segment (start 148.5 60) (end 148.5 61.675) (width 0.3) (layer "F.Cu") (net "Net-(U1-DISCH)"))
 (segment (start 137.5475 63.0875) (end 138.585 64.125) (width 0.3) (layer "F.Cu") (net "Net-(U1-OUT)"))
 (segment (start 136.4125 63.0875) (end 137.5475 63.0875) (width 0.3) (layer "F.Cu") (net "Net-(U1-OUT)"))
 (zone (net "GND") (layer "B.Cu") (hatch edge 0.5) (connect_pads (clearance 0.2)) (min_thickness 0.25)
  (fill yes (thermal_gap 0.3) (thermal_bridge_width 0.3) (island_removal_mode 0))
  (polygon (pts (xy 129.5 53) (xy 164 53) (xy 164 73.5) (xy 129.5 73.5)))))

